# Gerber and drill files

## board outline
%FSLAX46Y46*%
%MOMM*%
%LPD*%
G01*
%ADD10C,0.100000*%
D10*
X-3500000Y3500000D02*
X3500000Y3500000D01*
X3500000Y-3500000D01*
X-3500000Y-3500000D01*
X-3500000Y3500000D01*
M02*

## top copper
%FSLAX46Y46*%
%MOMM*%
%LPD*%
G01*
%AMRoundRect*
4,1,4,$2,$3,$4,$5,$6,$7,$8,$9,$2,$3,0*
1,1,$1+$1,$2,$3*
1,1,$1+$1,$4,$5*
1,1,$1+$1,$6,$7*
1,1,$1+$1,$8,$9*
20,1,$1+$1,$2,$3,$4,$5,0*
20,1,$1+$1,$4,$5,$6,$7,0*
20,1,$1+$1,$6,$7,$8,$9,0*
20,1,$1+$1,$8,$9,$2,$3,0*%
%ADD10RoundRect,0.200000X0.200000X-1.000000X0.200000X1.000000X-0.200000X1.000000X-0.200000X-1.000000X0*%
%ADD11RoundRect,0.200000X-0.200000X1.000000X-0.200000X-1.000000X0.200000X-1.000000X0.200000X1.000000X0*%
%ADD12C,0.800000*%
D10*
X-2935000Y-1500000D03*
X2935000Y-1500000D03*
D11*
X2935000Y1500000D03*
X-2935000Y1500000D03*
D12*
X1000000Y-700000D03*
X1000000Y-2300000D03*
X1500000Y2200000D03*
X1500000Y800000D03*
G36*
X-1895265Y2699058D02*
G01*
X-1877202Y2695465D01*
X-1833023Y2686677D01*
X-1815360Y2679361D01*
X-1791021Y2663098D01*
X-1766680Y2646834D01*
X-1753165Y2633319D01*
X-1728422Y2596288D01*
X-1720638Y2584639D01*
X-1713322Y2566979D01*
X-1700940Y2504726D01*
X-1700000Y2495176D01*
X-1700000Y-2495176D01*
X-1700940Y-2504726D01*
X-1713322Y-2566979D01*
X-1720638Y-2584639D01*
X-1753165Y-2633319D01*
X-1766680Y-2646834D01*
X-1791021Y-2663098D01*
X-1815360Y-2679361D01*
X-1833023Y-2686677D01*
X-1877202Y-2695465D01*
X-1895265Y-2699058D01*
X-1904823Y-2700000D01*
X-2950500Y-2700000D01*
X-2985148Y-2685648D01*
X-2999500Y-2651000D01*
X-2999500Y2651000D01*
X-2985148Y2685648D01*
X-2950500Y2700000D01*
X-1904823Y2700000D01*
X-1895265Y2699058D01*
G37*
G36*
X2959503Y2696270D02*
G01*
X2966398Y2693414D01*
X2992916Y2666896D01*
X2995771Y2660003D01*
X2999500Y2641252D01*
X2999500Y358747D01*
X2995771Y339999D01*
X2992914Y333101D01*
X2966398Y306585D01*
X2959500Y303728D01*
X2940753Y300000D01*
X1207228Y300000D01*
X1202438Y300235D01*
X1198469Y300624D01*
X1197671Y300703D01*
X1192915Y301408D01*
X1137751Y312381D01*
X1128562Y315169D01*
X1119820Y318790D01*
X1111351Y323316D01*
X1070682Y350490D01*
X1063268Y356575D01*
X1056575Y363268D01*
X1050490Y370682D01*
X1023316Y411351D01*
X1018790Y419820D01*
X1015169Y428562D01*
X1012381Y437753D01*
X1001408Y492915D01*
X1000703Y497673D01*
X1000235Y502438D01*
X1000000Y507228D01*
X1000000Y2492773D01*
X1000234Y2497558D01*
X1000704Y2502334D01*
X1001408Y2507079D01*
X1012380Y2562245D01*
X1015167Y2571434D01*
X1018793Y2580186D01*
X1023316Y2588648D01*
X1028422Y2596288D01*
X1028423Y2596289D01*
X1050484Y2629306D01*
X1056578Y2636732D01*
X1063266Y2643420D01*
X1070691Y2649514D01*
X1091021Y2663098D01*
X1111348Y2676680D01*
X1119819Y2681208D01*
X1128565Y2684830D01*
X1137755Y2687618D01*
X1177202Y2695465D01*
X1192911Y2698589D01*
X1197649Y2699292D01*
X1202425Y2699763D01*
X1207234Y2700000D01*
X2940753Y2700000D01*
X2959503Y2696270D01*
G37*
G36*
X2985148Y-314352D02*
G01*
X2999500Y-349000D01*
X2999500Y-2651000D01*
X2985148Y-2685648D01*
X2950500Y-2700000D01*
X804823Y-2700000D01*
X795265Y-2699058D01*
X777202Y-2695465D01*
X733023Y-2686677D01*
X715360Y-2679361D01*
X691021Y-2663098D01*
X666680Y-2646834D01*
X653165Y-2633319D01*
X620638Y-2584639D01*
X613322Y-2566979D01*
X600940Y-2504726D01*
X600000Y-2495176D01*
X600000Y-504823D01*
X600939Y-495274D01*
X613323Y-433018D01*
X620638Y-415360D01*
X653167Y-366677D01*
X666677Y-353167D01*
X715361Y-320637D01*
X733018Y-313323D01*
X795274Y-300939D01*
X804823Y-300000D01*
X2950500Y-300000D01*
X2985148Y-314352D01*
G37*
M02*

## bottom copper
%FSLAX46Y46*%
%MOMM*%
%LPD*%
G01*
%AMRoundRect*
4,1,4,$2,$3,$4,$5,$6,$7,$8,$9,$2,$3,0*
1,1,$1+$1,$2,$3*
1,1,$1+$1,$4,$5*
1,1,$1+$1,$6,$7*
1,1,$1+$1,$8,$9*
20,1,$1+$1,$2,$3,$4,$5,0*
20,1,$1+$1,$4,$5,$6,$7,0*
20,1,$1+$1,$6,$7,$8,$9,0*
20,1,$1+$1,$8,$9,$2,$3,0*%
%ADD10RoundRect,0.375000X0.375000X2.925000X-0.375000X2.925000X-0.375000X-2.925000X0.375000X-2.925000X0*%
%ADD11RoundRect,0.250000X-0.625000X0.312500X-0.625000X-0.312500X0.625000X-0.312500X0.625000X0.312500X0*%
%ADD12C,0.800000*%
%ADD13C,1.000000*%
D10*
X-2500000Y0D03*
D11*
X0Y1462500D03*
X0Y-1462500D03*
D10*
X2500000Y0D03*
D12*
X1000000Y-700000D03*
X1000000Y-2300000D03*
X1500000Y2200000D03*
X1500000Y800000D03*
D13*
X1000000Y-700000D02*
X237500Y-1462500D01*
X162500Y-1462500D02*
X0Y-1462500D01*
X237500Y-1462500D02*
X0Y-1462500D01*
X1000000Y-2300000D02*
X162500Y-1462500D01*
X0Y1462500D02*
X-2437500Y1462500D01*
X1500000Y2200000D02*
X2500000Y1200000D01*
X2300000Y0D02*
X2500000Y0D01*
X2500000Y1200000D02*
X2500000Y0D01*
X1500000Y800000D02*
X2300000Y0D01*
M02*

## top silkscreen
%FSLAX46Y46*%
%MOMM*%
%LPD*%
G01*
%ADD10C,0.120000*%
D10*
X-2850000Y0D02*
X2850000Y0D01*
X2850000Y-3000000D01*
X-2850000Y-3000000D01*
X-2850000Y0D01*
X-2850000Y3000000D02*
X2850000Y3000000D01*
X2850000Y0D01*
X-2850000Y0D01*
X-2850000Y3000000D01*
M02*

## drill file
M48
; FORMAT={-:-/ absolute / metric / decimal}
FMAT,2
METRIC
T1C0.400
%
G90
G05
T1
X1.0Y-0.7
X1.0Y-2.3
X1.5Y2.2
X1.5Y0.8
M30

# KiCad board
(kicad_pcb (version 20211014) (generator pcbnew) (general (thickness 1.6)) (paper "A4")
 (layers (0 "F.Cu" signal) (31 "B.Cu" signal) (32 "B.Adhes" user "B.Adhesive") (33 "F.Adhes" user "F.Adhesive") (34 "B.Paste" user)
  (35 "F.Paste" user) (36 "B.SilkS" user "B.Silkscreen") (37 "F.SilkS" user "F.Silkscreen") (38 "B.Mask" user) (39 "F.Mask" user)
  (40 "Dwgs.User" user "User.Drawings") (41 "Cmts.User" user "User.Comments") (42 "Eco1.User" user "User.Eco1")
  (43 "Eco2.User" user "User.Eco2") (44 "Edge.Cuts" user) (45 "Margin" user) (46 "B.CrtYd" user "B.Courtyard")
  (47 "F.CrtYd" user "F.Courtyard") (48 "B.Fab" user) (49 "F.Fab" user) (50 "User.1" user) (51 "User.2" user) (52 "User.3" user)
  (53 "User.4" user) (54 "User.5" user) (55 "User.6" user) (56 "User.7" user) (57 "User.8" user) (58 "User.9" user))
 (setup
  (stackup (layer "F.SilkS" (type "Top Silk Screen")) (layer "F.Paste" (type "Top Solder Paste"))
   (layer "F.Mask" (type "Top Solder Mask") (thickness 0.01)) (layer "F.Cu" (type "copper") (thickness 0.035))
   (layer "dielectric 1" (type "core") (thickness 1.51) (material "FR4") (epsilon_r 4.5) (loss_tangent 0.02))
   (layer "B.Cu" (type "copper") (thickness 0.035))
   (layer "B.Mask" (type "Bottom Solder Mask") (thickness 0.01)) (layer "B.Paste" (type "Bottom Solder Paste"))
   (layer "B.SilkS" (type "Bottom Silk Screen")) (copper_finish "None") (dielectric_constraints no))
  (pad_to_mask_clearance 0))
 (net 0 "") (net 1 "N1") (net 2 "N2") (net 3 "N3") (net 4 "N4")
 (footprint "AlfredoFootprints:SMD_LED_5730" (layer "F.Cu") (at 0 1.5)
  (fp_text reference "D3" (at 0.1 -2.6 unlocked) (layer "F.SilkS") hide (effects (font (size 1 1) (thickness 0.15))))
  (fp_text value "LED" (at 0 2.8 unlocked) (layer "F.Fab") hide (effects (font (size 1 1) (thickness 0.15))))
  (fp_rect (start -2.85 -1.5) (end 2.85 1.5) (layer "F.SilkS") (width 0.12) (fill none))
  (pad "1" smd roundrect (at -2.935 0 90) (size 2.4 0.8) (layers "F.Cu" "F.Paste" "F.Mask") (roundrect_rratio 0.25) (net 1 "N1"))
  (pad "2" smd roundrect (at 2.935 0 90) (size 2.4 0.8) (layers "F.Cu" "F.Paste" "F.Mask") (roundrect_rratio 0.25) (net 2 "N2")))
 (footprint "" (layer "F.Cu") (at -2.5 0)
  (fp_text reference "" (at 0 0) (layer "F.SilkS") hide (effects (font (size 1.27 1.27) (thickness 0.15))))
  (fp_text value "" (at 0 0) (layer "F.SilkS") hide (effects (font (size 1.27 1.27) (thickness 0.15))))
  (pad "1" smd roundrect (at 0 0 180) (size 1.5 6.6) (layers "B.Cu" "B.Paste" "B.Mask") (roundrect_rratio 0.25) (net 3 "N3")))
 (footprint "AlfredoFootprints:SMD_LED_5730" (layer "F.Cu") (at 0 -1.5 180)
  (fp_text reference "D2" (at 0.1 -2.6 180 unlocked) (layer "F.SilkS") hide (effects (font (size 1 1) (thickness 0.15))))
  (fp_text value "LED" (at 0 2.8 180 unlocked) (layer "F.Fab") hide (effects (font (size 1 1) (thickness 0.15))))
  (fp_rect (start -2.85 -1.5) (end 2.85 1.5) (layer "F.SilkS") (width 0.12) (fill none))
  (pad "1" smd roundrect (at -2.935 0 270) (size 2.4 0.8) (layers "F.Cu" "F.Paste" "F.Mask") (roundrect_rratio 0.25) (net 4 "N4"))
  (pad "2" smd roundrect (at 2.935 0 270) (size 2.4 0.8) (layers "F.Cu" "F.Paste" "F.Mask") (roundrect_rratio 0.25) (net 1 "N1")))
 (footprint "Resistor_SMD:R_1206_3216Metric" (layer "B.Cu") (at 0 0 -90)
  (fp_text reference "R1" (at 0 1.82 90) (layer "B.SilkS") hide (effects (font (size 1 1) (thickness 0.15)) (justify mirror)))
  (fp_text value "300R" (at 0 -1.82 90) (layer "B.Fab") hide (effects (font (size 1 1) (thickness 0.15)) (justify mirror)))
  (pad "1" smd roundrect (at -1.4625 0 270) (size 1.125 1.75) (layers "B.Cu" "B.Paste" "B.Mask") (roundrect_rratio 0.2222222222)
   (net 3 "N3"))
  (pad "2" smd roundrect (at 1.4625 0 270) (size 1.125 1.75) (layers "B.Cu" "B.Paste" "B.Mask") (roundrect_rratio 0.2222222222) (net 2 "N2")))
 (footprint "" (layer "B.Cu") (at 2.5 0 180)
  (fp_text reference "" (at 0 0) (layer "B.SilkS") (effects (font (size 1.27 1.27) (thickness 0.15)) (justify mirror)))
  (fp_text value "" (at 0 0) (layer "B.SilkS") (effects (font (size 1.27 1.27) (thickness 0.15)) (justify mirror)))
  (pad "1" smd roundrect (at 0 0 180) (size 1.5 6.6) (layers "B.Cu" "B.Paste" "B.Mask") (roundrect_rratio 0.25) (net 4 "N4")))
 (gr_rect (start -3.5 3.5) (end 3.5 -3.5) (layer "Edge.Cuts") (width 0.1) (fill none))
 (via (at 1 0.7) (size 0.8) (drill 0.4) (layers "F.Cu" "B.Cu") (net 2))
 (via (at 1 2.3) (size 0.8) (drill 0.4) (layers "F.Cu" "B.Cu") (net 2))
 (segment (start 1 0.7) (end 0.2375 1.4625) (width 1) (layer "B.Cu") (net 2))
 (segment (start 0.1625 1.4625) (end 0 1.4625) (width 1) (layer "B.Cu") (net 2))
 (segment (start 0.2375 1.4625) (end 0 1.4625) (width 1) (layer "B.Cu") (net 2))
 (segment (start 1 2.3) (end 0.1625 1.4625) (width 1) (layer "B.Cu") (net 2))
 (segment (start 0 -1.4625) (end -2.4375 -1.4625) (width 1) (layer "B.Cu") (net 3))
 (via (at 1.5 -2.2) (size 0.8) (drill 0.4) (layers "F.Cu" "B.Cu") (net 4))
 (via (at 1.5 -0.8) (size 0.8) (drill 0.4) (layers "F.Cu" "B.Cu") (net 4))
 (segment (start 1.5 -2.2) (end 2.5 -1.2) (width 1) (layer "B.Cu") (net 4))
 (segment (start 2.3 0) (end 2.5 0) (width 1) (layer "B.Cu") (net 4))
 (segment (start 2.5 -1.2) (end 2.5 0) (width 1) (layer "B.Cu") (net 4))
 (segment (start 1.5 -0.8) (end 2.3 0) (width 1) (layer "B.Cu") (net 4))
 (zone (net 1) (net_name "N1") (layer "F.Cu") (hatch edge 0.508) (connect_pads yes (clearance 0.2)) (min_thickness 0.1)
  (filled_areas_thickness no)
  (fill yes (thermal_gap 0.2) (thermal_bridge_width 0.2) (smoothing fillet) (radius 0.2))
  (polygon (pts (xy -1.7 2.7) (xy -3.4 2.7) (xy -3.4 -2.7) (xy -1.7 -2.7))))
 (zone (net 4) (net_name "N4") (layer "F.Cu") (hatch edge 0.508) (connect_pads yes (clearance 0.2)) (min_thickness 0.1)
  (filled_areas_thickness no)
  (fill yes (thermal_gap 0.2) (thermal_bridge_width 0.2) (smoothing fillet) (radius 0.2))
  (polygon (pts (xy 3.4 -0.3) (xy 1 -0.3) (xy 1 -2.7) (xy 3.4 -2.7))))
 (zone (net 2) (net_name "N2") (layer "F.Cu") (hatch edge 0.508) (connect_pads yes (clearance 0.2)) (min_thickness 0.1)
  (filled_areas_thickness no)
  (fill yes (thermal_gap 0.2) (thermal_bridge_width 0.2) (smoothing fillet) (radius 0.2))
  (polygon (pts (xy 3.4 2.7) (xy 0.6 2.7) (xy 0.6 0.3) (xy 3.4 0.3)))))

